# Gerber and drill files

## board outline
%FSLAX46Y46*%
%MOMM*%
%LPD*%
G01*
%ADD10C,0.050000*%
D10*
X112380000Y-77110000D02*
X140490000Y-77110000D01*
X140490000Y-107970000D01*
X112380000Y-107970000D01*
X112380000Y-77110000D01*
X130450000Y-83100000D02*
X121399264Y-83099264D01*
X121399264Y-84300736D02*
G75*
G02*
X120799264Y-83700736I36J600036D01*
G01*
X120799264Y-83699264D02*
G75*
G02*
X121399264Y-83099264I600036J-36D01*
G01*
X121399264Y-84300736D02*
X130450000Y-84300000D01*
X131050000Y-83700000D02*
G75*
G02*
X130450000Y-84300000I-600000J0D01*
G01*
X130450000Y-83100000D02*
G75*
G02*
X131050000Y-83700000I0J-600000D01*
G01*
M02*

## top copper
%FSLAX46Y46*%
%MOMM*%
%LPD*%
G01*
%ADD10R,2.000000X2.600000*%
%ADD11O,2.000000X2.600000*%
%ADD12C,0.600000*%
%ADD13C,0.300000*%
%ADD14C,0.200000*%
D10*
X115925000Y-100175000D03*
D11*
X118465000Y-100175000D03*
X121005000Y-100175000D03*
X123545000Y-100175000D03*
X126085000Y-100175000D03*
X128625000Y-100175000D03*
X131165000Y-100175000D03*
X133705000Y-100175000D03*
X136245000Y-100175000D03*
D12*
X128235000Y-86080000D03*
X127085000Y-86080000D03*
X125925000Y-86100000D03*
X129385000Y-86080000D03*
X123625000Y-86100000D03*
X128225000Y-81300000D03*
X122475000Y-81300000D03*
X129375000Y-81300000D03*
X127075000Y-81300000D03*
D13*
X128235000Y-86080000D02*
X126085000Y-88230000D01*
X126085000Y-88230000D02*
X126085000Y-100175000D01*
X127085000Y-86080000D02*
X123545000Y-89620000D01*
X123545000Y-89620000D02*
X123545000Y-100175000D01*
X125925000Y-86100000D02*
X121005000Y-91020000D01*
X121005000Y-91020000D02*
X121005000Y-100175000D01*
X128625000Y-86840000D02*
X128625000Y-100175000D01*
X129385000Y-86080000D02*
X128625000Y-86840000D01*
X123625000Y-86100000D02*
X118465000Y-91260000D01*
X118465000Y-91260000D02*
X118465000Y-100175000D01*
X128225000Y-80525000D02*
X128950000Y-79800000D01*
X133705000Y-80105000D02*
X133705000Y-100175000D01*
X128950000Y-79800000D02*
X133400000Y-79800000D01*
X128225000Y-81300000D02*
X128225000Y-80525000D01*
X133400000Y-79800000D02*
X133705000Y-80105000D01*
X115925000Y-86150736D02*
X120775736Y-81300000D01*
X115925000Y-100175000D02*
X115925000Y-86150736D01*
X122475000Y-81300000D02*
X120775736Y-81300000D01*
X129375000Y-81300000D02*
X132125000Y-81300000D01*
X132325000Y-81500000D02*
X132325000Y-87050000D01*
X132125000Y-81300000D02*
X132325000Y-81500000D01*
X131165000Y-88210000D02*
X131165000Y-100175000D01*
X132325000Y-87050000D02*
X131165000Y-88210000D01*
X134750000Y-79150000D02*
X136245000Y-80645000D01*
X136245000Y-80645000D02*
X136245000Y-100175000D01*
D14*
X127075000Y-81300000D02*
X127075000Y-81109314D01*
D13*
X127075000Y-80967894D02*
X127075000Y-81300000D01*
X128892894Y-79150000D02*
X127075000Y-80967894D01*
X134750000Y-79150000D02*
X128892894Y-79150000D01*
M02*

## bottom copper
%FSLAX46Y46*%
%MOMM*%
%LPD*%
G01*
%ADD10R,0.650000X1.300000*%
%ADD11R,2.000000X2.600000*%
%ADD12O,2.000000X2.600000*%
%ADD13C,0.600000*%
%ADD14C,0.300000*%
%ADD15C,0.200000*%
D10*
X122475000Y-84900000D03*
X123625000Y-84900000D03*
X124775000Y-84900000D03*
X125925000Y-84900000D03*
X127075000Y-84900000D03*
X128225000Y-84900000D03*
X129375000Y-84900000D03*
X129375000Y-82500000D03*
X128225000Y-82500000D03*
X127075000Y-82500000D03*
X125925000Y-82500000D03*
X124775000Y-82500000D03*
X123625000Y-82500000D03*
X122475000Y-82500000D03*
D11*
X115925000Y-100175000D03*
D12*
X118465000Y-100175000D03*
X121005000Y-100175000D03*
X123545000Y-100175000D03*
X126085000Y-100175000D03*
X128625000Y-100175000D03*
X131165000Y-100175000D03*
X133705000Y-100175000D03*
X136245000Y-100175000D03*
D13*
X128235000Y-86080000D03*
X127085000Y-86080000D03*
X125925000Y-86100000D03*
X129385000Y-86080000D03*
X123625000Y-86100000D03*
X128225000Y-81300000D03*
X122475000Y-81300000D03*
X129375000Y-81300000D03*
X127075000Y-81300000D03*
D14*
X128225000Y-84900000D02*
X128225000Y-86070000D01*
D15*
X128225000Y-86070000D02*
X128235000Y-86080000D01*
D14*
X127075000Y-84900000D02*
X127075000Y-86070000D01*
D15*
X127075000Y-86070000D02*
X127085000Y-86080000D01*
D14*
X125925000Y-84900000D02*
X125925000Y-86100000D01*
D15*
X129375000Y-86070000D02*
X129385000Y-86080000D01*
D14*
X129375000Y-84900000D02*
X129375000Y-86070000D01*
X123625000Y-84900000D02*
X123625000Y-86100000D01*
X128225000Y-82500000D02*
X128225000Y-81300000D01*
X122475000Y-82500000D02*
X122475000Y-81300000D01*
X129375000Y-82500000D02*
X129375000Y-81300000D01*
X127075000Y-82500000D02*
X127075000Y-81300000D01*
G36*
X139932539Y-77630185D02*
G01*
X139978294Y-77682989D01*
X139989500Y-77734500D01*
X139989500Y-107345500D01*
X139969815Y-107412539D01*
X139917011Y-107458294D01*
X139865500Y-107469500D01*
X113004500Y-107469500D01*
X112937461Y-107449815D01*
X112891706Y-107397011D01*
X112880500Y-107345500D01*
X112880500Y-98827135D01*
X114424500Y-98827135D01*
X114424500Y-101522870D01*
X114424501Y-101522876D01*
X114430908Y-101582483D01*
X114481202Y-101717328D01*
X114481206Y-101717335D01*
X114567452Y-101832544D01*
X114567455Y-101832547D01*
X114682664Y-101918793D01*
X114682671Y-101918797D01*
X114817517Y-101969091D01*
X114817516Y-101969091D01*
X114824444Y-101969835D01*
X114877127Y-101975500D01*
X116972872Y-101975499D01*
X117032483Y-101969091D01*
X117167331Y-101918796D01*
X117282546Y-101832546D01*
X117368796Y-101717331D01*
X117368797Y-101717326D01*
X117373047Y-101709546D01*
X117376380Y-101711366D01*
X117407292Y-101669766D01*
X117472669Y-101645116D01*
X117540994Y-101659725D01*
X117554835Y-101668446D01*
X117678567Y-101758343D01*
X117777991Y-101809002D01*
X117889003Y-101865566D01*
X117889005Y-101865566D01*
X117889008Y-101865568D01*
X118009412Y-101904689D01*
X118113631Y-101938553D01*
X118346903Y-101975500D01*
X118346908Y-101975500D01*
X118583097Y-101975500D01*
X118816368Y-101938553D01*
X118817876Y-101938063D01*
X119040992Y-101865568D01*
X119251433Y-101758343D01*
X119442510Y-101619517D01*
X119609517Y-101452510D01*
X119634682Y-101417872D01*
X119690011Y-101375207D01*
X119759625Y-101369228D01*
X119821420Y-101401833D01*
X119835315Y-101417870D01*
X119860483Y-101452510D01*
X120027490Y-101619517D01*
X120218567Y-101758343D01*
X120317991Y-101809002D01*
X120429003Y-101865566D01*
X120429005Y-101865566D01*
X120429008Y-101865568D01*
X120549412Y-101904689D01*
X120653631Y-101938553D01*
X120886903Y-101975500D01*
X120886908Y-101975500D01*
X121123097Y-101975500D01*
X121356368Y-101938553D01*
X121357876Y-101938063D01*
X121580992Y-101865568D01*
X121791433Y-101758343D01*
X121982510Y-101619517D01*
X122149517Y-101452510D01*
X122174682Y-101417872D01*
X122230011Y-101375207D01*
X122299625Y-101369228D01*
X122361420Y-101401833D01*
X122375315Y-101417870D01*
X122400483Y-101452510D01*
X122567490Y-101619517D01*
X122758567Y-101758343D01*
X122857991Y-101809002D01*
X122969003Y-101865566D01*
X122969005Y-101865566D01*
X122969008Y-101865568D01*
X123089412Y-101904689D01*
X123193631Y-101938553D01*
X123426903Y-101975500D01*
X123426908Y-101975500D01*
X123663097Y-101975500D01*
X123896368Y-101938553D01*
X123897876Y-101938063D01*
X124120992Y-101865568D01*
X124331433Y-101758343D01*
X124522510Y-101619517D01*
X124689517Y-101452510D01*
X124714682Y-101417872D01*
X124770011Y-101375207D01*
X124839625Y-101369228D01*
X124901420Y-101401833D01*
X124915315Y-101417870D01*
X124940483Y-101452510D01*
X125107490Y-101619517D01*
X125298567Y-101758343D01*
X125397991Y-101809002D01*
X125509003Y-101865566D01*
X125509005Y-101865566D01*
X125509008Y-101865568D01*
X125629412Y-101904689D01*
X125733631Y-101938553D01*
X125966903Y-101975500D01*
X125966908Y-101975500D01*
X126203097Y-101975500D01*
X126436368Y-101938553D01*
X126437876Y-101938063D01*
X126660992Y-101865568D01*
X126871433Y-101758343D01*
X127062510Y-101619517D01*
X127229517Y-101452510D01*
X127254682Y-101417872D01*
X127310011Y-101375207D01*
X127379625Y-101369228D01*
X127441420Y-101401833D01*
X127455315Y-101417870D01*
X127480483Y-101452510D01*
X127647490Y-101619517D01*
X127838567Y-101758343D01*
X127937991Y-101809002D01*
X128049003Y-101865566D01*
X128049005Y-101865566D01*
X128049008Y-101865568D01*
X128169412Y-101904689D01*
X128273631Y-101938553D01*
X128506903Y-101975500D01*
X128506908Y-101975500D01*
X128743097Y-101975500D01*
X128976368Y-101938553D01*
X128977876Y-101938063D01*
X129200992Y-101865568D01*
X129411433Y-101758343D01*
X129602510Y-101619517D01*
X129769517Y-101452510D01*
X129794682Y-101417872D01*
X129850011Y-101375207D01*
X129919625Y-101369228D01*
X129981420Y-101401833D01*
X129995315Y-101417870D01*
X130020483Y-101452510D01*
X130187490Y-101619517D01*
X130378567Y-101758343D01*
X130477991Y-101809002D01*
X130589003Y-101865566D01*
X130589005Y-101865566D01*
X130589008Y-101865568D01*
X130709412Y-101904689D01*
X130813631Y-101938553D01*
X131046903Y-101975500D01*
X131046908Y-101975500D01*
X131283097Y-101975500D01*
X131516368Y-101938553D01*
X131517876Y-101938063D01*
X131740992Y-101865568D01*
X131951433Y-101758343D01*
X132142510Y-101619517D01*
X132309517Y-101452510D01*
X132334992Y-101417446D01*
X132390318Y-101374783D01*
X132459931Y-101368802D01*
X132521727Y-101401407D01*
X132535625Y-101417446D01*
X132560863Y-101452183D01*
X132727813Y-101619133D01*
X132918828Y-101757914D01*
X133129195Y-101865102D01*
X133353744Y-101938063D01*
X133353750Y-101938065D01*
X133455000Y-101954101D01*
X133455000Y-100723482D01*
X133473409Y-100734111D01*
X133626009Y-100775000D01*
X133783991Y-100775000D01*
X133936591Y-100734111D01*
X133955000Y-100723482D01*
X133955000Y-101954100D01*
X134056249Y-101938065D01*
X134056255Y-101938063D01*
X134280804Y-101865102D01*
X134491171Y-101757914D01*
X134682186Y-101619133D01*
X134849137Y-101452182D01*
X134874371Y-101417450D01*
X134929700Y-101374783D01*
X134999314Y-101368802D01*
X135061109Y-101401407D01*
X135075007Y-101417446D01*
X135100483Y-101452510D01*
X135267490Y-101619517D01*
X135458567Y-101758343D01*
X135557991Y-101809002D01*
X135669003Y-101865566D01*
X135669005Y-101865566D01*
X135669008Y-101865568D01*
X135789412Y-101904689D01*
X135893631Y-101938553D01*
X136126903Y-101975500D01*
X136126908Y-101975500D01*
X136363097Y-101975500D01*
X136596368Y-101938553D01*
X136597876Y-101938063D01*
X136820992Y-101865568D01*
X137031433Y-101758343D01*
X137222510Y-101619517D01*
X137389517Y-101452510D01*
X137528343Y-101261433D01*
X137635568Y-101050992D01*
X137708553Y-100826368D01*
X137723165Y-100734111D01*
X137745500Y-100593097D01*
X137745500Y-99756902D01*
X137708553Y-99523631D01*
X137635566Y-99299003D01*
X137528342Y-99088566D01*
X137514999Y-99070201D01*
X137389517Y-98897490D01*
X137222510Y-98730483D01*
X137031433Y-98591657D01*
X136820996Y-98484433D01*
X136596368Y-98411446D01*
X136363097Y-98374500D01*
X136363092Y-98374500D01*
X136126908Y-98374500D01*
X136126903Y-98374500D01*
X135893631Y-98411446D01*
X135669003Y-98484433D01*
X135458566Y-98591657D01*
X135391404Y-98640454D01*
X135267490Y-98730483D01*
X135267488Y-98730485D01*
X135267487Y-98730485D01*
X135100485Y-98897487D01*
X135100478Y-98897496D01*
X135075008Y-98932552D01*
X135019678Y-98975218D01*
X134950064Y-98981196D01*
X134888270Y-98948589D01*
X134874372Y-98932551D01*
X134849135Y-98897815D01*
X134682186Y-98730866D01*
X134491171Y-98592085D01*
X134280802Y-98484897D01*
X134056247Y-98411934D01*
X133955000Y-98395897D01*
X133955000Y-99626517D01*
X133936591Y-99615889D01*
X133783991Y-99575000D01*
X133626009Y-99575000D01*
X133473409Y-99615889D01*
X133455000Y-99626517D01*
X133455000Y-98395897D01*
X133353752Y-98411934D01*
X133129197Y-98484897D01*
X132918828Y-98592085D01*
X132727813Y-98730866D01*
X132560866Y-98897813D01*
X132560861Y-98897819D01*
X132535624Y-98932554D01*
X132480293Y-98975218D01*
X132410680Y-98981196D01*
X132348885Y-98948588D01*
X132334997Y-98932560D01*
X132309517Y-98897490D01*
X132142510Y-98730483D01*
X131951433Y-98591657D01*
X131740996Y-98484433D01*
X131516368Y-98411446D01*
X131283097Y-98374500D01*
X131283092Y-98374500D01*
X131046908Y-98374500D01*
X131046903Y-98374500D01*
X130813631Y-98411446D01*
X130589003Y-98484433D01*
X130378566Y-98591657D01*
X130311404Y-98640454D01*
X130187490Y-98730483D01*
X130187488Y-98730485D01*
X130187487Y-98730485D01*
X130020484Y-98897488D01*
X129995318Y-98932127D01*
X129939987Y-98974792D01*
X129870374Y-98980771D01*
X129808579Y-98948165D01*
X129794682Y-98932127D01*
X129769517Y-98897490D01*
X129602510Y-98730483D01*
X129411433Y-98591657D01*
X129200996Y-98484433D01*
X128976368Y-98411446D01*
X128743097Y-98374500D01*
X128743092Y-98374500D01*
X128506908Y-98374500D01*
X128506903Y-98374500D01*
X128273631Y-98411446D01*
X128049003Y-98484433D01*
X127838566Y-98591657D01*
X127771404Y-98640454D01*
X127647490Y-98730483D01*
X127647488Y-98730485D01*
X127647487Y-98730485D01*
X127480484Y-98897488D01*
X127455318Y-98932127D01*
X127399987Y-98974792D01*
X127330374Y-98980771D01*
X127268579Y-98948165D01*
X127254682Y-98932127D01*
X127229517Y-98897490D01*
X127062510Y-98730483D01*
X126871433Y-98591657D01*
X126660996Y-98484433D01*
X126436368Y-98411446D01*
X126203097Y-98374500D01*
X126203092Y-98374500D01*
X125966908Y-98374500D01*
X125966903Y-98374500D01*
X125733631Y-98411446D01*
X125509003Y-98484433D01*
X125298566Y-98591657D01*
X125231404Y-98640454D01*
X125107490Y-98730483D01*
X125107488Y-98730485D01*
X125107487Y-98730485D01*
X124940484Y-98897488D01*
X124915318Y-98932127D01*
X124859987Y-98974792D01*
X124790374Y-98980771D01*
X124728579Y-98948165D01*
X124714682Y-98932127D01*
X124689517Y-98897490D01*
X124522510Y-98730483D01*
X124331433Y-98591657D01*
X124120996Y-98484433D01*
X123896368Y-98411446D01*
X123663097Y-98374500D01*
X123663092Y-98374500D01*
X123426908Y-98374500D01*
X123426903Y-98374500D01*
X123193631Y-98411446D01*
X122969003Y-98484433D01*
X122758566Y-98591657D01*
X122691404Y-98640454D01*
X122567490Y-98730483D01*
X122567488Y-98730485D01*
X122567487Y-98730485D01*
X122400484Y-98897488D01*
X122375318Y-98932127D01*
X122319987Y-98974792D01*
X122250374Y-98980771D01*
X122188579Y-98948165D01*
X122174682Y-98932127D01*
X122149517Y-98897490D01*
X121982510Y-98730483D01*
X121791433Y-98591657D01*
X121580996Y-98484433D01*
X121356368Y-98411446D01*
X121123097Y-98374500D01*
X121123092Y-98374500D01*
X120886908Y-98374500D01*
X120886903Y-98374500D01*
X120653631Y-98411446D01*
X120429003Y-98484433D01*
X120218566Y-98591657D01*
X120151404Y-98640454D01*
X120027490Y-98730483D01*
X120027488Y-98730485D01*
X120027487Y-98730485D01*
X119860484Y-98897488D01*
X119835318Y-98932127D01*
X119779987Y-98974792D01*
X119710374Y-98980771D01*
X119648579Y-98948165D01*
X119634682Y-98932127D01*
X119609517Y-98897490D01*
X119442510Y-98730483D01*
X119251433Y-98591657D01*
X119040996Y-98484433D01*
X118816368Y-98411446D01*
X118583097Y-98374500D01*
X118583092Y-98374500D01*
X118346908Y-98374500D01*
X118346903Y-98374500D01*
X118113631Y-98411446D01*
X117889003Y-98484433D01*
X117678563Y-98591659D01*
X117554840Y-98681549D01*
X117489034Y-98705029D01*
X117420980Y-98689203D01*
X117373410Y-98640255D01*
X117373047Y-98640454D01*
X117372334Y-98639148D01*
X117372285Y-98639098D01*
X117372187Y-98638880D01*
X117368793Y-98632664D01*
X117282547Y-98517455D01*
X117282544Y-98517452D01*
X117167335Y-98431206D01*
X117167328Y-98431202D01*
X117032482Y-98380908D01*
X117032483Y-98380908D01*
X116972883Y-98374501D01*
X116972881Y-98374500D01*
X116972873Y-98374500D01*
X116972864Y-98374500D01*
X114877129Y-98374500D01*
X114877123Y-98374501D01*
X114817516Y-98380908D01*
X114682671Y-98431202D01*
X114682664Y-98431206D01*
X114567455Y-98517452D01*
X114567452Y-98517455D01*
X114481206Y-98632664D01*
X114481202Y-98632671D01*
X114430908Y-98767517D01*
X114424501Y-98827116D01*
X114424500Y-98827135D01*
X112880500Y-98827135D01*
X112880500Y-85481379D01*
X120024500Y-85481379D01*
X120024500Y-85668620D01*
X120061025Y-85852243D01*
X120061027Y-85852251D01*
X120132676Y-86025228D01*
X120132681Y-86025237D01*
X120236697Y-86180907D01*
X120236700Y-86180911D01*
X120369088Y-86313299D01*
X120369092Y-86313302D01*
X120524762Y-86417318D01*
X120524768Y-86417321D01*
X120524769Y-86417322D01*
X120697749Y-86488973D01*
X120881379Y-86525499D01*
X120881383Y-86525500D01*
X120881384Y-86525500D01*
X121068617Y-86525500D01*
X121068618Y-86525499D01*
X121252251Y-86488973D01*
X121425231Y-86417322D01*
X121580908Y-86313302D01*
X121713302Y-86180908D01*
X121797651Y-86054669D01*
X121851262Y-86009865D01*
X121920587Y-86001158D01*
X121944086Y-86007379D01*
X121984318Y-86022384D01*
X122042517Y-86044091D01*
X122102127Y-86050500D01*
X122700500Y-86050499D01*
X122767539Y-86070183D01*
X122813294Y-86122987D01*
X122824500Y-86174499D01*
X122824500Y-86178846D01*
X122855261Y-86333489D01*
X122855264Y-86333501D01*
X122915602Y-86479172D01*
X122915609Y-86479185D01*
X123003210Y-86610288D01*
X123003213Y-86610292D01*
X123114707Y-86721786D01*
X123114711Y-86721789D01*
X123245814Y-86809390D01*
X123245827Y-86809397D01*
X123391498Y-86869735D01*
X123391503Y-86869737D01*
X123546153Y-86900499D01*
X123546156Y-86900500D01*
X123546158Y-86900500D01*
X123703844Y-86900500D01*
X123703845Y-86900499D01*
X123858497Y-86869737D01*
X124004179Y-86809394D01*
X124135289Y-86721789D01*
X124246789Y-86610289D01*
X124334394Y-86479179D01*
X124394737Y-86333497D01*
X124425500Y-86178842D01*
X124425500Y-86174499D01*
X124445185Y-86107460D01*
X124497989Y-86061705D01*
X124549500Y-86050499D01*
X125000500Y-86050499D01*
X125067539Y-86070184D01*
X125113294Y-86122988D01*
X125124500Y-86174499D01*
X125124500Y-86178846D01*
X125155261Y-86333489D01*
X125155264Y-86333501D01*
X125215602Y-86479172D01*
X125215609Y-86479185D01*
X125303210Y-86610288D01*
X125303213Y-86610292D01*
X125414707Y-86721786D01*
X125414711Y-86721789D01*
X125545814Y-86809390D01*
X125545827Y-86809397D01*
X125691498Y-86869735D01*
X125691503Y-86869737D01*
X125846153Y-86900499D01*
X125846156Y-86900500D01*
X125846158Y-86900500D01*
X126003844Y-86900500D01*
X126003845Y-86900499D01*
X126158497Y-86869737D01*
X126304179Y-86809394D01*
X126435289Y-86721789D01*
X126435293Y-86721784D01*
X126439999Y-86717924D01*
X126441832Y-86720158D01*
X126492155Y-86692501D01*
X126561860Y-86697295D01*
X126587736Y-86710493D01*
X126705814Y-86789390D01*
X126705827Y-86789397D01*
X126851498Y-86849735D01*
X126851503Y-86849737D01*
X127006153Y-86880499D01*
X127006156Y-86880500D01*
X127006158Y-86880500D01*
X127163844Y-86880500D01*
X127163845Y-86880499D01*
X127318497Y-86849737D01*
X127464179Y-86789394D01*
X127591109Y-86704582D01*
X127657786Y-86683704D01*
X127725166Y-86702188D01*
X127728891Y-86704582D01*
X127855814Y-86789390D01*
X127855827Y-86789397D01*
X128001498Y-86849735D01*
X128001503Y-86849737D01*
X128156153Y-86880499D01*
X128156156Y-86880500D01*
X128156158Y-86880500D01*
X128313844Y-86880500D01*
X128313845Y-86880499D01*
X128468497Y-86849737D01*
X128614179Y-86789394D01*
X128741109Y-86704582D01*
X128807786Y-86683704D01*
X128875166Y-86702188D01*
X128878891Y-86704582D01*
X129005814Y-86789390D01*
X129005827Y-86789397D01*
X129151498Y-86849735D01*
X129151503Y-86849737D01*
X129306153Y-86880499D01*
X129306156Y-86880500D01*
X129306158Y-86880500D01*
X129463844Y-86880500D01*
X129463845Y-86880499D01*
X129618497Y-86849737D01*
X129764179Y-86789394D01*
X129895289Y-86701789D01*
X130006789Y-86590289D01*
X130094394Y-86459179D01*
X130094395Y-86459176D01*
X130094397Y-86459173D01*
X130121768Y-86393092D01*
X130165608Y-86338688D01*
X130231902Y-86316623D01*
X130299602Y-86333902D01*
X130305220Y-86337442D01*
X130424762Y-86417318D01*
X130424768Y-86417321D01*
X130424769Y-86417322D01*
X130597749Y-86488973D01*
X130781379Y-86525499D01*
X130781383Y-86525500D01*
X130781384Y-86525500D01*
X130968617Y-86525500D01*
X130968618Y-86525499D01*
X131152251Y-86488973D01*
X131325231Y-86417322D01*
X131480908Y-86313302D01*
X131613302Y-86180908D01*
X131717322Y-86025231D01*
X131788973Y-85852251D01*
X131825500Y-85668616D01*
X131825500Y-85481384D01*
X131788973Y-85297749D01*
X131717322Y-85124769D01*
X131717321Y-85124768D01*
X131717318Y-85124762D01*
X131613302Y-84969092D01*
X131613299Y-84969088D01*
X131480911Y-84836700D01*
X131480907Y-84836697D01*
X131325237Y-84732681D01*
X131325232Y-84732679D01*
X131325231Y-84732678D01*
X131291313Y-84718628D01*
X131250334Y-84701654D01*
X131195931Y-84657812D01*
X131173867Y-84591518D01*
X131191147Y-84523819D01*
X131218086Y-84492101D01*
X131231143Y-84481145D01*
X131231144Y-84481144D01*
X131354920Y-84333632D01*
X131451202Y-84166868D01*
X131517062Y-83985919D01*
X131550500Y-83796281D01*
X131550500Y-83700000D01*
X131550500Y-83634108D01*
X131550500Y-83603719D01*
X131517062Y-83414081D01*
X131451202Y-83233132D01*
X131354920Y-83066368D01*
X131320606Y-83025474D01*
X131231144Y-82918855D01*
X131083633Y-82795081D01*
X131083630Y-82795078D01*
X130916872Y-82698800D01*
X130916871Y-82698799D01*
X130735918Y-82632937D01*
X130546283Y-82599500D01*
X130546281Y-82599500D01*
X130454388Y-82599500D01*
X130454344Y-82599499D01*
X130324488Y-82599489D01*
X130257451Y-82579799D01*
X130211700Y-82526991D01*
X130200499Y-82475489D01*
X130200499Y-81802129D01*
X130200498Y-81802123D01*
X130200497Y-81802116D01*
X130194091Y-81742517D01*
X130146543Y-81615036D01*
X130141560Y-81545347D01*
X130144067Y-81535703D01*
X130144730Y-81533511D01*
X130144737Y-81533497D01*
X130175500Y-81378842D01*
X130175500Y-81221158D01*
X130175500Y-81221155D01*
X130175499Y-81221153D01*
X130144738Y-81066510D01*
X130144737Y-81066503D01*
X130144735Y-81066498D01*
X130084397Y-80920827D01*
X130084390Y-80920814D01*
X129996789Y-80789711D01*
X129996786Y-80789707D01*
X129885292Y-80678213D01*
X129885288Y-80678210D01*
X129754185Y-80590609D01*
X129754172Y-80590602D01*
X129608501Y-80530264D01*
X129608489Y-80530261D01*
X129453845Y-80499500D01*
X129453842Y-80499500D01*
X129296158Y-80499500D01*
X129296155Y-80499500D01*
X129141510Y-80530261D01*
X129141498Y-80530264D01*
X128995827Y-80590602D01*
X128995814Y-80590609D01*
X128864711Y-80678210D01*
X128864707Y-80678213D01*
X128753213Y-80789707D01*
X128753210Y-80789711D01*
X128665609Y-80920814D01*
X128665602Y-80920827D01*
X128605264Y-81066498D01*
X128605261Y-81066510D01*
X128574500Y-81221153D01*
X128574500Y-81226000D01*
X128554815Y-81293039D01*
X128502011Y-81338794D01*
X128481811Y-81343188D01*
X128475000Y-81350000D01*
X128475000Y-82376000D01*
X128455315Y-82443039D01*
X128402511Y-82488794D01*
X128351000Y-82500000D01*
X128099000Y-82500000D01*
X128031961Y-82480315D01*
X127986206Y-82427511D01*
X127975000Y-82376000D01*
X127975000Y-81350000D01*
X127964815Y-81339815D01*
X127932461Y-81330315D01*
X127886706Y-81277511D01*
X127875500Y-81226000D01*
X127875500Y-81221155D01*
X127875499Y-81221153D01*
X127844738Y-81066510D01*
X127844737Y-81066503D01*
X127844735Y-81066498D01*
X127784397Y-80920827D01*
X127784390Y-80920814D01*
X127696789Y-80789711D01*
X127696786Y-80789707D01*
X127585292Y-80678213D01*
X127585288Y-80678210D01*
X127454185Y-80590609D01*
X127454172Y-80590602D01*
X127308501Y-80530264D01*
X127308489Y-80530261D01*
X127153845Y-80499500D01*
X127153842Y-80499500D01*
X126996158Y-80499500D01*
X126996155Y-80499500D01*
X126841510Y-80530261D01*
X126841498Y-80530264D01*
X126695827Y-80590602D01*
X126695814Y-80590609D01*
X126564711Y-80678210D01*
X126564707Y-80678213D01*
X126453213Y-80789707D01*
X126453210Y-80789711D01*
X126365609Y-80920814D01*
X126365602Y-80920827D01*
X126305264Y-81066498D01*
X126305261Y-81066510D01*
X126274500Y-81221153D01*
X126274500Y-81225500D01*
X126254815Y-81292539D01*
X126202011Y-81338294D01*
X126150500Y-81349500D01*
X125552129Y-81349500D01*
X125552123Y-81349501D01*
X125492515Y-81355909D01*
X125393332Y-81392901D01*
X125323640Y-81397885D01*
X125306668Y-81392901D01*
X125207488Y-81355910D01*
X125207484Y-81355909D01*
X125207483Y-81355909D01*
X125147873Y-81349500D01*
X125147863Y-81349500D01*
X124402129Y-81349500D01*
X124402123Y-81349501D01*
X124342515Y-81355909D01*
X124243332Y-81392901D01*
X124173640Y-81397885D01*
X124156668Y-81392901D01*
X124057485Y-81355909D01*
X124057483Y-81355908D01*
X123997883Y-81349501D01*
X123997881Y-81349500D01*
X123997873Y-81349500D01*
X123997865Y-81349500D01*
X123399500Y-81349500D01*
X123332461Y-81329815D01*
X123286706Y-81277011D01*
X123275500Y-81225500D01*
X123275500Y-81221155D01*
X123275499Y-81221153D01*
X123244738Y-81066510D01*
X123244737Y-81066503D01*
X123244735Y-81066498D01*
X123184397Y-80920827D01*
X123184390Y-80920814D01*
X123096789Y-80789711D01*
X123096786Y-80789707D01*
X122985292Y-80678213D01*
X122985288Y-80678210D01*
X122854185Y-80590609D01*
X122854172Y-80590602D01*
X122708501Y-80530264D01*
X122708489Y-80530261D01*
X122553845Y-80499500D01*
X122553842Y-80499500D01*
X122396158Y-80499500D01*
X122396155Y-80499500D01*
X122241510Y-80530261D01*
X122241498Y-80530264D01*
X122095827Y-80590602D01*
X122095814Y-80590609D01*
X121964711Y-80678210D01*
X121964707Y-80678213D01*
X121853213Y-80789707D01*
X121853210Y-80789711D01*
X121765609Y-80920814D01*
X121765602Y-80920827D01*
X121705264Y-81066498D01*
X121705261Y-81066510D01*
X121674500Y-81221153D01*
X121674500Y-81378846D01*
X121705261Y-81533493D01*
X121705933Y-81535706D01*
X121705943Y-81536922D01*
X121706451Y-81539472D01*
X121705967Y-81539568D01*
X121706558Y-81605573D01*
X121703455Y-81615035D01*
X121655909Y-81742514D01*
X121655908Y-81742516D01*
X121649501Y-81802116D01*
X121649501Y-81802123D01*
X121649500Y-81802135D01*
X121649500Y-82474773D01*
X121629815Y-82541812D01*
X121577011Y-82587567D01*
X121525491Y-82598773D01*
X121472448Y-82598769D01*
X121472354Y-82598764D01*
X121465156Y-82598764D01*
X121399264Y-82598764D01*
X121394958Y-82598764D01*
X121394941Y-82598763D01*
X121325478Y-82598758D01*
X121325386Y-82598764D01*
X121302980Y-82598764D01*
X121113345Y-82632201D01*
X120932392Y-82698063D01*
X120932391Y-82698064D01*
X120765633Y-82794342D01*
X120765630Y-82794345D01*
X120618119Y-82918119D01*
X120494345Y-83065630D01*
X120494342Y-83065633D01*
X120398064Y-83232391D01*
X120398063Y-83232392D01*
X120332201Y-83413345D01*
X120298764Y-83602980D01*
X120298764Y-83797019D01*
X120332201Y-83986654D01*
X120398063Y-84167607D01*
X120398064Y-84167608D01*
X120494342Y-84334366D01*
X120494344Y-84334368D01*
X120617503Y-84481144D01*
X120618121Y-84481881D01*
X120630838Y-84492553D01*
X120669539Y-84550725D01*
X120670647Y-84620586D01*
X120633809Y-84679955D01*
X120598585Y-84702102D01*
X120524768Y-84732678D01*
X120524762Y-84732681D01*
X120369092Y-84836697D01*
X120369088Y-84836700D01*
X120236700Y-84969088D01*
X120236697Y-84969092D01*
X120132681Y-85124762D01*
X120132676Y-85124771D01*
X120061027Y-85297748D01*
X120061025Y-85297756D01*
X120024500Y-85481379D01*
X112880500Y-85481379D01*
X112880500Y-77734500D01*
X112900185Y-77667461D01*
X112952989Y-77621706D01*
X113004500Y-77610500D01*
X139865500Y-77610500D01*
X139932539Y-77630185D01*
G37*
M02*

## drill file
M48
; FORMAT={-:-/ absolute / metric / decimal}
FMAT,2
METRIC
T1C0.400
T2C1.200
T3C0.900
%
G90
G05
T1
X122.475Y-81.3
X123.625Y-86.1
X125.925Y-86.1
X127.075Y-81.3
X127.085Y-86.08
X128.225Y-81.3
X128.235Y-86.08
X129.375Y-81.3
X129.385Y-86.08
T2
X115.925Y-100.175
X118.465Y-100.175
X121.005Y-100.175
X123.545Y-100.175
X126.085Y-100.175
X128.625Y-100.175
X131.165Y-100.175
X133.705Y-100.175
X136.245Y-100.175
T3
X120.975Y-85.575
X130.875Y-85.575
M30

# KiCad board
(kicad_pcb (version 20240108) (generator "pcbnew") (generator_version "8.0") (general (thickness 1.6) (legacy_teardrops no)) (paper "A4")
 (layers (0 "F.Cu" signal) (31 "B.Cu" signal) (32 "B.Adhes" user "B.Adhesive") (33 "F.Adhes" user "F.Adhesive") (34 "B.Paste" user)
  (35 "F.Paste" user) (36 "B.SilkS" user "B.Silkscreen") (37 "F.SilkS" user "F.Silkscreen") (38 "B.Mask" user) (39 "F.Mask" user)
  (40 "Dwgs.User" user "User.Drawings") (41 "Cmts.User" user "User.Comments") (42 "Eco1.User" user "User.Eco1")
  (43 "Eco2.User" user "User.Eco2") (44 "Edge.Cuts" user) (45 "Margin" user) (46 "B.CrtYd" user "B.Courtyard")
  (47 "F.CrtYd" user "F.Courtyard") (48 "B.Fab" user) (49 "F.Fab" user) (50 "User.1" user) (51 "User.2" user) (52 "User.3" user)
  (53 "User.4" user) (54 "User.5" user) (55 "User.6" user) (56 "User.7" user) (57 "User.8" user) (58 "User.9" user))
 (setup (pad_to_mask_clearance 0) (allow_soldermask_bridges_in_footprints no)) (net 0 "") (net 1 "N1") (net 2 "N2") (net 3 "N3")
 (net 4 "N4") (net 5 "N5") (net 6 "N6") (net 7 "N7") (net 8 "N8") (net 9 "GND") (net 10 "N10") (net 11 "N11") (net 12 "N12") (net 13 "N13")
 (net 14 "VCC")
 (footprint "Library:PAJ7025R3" (layer "F.Cu") (at 125.925 83.7)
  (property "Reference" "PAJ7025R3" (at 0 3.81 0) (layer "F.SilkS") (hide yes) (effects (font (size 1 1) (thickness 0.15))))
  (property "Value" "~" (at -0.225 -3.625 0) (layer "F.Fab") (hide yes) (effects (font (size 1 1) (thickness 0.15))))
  (pad "" np_thru_hole oval (at -4.95 1.875) (size 0.9 0.9) (drill 0.9) (layers "F&B.Cu"))
  (pad "" np_thru_hole oval (at 4.95 1.875) (size 0.9 0.9) (drill 0.9) (layers "*.Cu"))
  (pad "1" smd rect (at -3.45 1.2) (size 0.65 1.3) (layers "B.Cu" "B.Paste" "B.Mask") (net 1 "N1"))
  (pad "2" smd rect (at -2.3 1.2) (size 0.65 1.3) (layers "B.Cu" "B.Paste" "B.Mask") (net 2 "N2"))
  (pad "3" smd rect (at -1.15 1.2) (size 0.65 1.3) (layers "B.Cu" "B.Paste" "B.Mask") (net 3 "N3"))
  (pad "4" smd rect (at 0 1.2) (size 0.65 1.3) (layers "B.Cu" "B.Paste" "B.Mask") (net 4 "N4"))
  (pad "5" smd rect (at 1.15 1.2) (size 0.65 1.3) (layers "B.Cu" "B.Paste" "B.Mask") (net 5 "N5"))
  (pad "6" smd rect (at 2.3 1.2) (size 0.65 1.3) (layers "B.Cu" "B.Paste" "B.Mask") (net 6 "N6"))
  (pad "7" smd rect (at 3.45 1.2) (size 0.65 1.3) (layers "B.Cu" "B.Paste" "B.Mask") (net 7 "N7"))
  (pad "8" smd rect (at 3.45 -1.2) (size 0.65 1.3) (layers "B.Cu" "B.Paste" "B.Mask") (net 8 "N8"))
  (pad "9" smd rect (at 2.3 -1.2) (size 0.65 1.3) (layers "B.Cu" "B.Paste" "B.Mask") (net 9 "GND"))
  (pad "10" smd rect (at 1.15 -1.2) (size 0.65 1.3) (layers "B.Cu" "B.Paste" "B.Mask") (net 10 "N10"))
  (pad "11" smd rect (at 0 -1.2) (size 0.65 1.3) (layers "B.Cu" "B.Paste" "B.Mask") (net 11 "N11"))
  (pad "12" smd rect (at -1.15 -1.2) (size 0.65 1.3) (layers "B.Cu" "B.Paste" "B.Mask") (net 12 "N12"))
  (pad "13" smd rect (at -2.3 -1.2) (size 0.65 1.3) (layers "B.Cu" "B.Paste" "B.Mask") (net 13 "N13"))
  (pad "14" smd rect (at -3.45 -1.2) (size 0.65 1.3) (layers "B.Cu" "B.Paste" "B.Mask") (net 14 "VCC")))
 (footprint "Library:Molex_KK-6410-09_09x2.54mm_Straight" (layer "F.Cu") (at 115.925 100.175)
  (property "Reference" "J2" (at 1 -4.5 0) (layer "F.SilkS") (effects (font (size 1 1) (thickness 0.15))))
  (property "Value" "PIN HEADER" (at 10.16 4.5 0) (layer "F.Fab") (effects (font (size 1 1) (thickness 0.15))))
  (pad "1" thru_hole rect (at 0 0) (size 2 2.6) (drill 1.2) (layers "*.Cu" "*.Mask") (remove_unused_layers yes) (keep_end_layers yes)
   (zone_layer_connections) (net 14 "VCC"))
  (pad "2" thru_hole oval (at 2.54 0) (size 2 2.6) (drill 1.2) (layers "*.Cu" "*.Mask") (remove_unused_layers yes) (keep_end_layers yes)
   (zone_layer_connections) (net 2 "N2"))
  (pad "3" thru_hole oval (at 5.08 0) (size 2 2.6) (drill 1.2) (layers "*.Cu" "*.Mask") (remove_unused_layers yes) (keep_end_layers yes)
   (zone_layer_connections) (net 4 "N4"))
  (pad "4" thru_hole oval (at 7.62 0) (size 2 2.6) (drill 1.2) (layers "*.Cu" "*.Mask") (remove_unused_layers yes) (keep_end_layers yes)
   (zone_layer_connections) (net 5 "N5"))
  (pad "5" thru_hole oval (at 10.16 0) (size 2 2.6) (drill 1.2) (layers "*.Cu" "*.Mask") (remove_unused_layers yes) (keep_end_layers yes)
   (zone_layer_connections) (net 6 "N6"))
  (pad "6" thru_hole oval (at 12.7 0) (size 2 2.6) (drill 1.2) (layers "*.Cu" "*.Mask") (remove_unused_layers yes) (keep_end_layers yes)
   (zone_layer_connections) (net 7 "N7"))
  (pad "7" thru_hole oval (at 15.24 0) (size 2 2.6) (drill 1.2) (layers "*.Cu" "*.Mask") (remove_unused_layers yes) (keep_end_layers yes)
   (zone_layer_connections) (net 8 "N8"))
  (pad "8" thru_hole oval (at 17.78 0) (size 2 2.6) (drill 1.2) (layers "*.Cu" "*.Mask") (remove_unused_layers yes) (keep_end_layers yes)
   (zone_layer_connections) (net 9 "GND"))
  (pad "9" thru_hole oval (at 20.32 0) (size 2 2.6) (drill 1.2) (layers "*.Cu" "*.Mask") (remove_unused_layers yes) (keep_end_layers yes)
   (zone_layer_connections) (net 10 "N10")))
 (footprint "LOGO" (layer "F.Cu") (at 115.384989 81.940094)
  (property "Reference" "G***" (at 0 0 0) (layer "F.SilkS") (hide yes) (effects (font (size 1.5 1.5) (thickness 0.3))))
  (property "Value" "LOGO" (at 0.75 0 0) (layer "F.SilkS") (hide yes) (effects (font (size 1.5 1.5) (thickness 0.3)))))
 (gr_rect (start 112.38 77.11) (end 140.49 107.97) (stroke (width 0.05) (type default)) (fill none) (layer "Edge.Cuts"))
 (gr_line (start 130.45 83.1) (end 121.399264 83.099264) (stroke (width 0.05) (type default)) (layer "Edge.Cuts"))
 (gr_arc (start 121.399264 84.300736) (mid 120.975 84.125) (end 120.799264 83.700736) (stroke (width 0.05) (type default))
  (layer "Edge.Cuts"))
 (gr_arc (start 120.799264 83.699264) (mid 120.975 83.275) (end 121.399264 83.099264) (stroke (width 0.05) (type default))
  (layer "Edge.Cuts"))
 (gr_line (start 121.399264 84.300736) (end 130.45 84.3) (stroke (width 0.05) (type default)) (layer "Edge.Cuts"))
 (gr_arc (start 131.05 83.7) (mid 130.874264 84.124264) (end 130.45 84.3) (stroke (width 0.05) (type default)) (layer "Edge.Cuts"))
 (gr_arc (start 130.45 83.1) (mid 130.874264 83.275736) (end 131.05 83.7) (stroke (width 0.05) (type default)) (layer "Edge.Cuts"))
 (segment (start 128.235 86.08) (end 126.085 88.23) (width 0.3) (layer "F.Cu") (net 6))
 (segment (start 126.085 88.23) (end 126.085 100.175) (width 0.3) (layer "F.Cu") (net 6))
 (via (at 128.235 86.08) (size 0.6) (drill 0.4) (layers "F.Cu" "B.Cu") (remove_unused_layers yes) (keep_end_layers yes) (free yes)
  (zone_layer_connections) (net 6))
 (segment (start 128.225 84.9) (end 128.225 86.07) (width 0.3) (layer "B.Cu") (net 6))
 (segment (start 128.225 86.07) (end 128.235 86.08) (width 0.2) (layer "B.Cu") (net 6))
 (segment (start 127.085 86.08) (end 123.545 89.62) (width 0.3) (layer "F.Cu") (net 5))
 (segment (start 123.545 89.62) (end 123.545 100.175) (width 0.3) (layer "F.Cu") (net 5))
 (via (at 127.085 86.08) (size 0.6) (drill 0.4) (layers "F.Cu" "B.Cu") (remove_unused_layers yes) (keep_end_layers yes) (free yes)
  (zone_layer_connections) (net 5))
 (segment (start 127.075 84.9) (end 127.075 86.07) (width 0.3) (layer "B.Cu") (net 5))
 (segment (start 127.075 86.07) (end 127.085 86.08) (width 0.2) (layer "B.Cu") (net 5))
 (segment (start 125.925 86.1) (end 121.005 91.02) (width 0.3) (layer "F.Cu") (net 4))
 (segment (start 121.005 91.02) (end 121.005 100.175) (width 0.3) (layer "F.Cu") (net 4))
 (via (at 125.925 86.1) (size 0.6) (drill 0.4) (layers "F.Cu" "B.Cu") (remove_unused_layers yes) (keep_end_layers yes) (free yes)
  (zone_layer_connections) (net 4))
 (segment (start 125.925 84.9) (end 125.925 86.1) (width 0.3) (layer "B.Cu") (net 4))
 (segment (start 128.625 86.84) (end 128.625 100.175) (width 0.3) (layer "F.Cu") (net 7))
 (segment (start 129.385 86.08) (end 128.625 86.84) (width 0.3) (layer "F.Cu") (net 7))
 (via (at 129.385 86.08) (size 0.6) (drill 0.4) (layers "F.Cu" "B.Cu") (remove_unused_layers yes) (keep_end_layers yes) (free yes)
  (zone_layer_connections) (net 7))
 (segment (start 129.375 86.07) (end 129.385 86.08) (width 0.2) (layer "B.Cu") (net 7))
 (segment (start 129.375 84.9) (end 129.375 86.07) (width 0.3) (layer "B.Cu") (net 7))
 (segment (start 123.625 86.1) (end 118.465 91.26) (width 0.3) (layer "F.Cu") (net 2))
 (segment (start 118.465 91.26) (end 118.465 100.175) (width 0.3) (layer "F.Cu") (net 2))
 (via (at 123.625 86.1) (size 0.6) (drill 0.4) (layers "F.Cu" "B.Cu") (remove_unused_layers yes) (keep_end_layers yes) (free yes)
  (zone_layer_connections) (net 2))
 (segment (start 123.625 84.9) (end 123.625 86.1) (width 0.3) (layer "B.Cu") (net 2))
 (segment (start 128.225 80.525) (end 128.95 79.8) (width 0.3) (layer "F.Cu") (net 9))
 (segment (start 133.705 80.105) (end 133.705 100.175) (width 0.3) (layer "F.Cu") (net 9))
 (segment (start 128.95 79.8) (end 133.4 79.8) (width 0.3) (layer "F.Cu") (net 9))
 (segment (start 128.225 81.3) (end 128.225 80.525) (width 0.3) (layer "F.Cu") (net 9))
 (segment (start 133.4 79.8) (end 133.705 80.105) (width 0.3) (layer "F.Cu") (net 9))
 (via (at 128.225 81.3) (size 0.6) (drill 0.4) (layers "F.Cu" "B.Cu") (remove_unused_layers yes) (keep_end_layers yes) (free yes)
  (zone_layer_connections) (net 9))
 (segment (start 128.225 82.5) (end 128.225 81.3) (width 0.3) (layer "B.Cu") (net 9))
 (segment (start 115.925 86.150736) (end 120.775736 81.3) (width 0.3) (layer "F.Cu") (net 14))
 (segment (start 115.925 100.175) (end 115.925 86.150736) (width 0.3) (layer "F.Cu") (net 14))
 (segment (start 122.475 81.3) (end 120.775736 81.3) (width 0.3) (layer "F.Cu") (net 14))
 (via (at 122.475 81.3) (size 0.6) (drill 0.4) (layers "F.Cu" "B.Cu") (remove_unused_layers yes) (keep_end_layers yes) (free yes)
  (zone_layer_connections) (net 14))
 (segment (start 122.475 82.5) (end 122.475 81.3) (width 0.3) (layer "B.Cu") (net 14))
 (segment (start 129.375 81.3) (end 132.125 81.3) (width 0.3) (layer "F.Cu") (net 8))
 (segment (start 132.325 81.5) (end 132.325 87.05) (width 0.3) (layer "F.Cu") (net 8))
 (segment (start 132.125 81.3) (end 132.325 81.5) (width 0.3) (layer "F.Cu") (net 8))
 (segment (start 131.165 88.21) (end 131.165 100.175) (width 0.3) (layer "F.Cu") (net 8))
 (segment (start 132.325 87.05) (end 131.165 88.21) (width 0.3) (layer "F.Cu") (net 8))
 (via (at 129.375 81.3) (size 0.6) (drill 0.4) (layers "F.Cu" "B.Cu") (remove_unused_layers yes) (keep_end_layers yes) (free yes)
  (zone_layer_connections) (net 8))
 (segment (start 129.375 82.5) (end 129.375 81.3) (width 0.3) (layer "B.Cu") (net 8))
 (segment (start 134.75 79.15) (end 136.245 80.645) (width 0.3) (layer "F.Cu") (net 10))
 (segment (start 136.245 80.645) (end 136.245 100.175) (width 0.3) (layer "F.Cu") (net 10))
 (segment (start 127.075 81.3) (end 127.075 81.109314) (width 0.2) (layer "F.Cu") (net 10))
 (segment (start 127.075 80.967894) (end 127.075 81.3) (width 0.3) (layer "F.Cu") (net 10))
 (segment (start 128.892894 79.15) (end 127.075 80.967894) (width 0.3) (layer "F.Cu") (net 10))
 (segment (start 134.75 79.15) (end 128.892894 79.15) (width 0.3) (layer "F.Cu") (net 10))
 (via (at 127.075 81.3) (size 0.6) (drill 0.4) (layers "F.Cu" "B.Cu") (remove_unused_layers yes) (keep_end_layers yes) (free yes)
  (zone_layer_connections) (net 10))
 (segment (start 127.075 82.5) (end 127.075 81.3) (width 0.3) (layer "B.Cu") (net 10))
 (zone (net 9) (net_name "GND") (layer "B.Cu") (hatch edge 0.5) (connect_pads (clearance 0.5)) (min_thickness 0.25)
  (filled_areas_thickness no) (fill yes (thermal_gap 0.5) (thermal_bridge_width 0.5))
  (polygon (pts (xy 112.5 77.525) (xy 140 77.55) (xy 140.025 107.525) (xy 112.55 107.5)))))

